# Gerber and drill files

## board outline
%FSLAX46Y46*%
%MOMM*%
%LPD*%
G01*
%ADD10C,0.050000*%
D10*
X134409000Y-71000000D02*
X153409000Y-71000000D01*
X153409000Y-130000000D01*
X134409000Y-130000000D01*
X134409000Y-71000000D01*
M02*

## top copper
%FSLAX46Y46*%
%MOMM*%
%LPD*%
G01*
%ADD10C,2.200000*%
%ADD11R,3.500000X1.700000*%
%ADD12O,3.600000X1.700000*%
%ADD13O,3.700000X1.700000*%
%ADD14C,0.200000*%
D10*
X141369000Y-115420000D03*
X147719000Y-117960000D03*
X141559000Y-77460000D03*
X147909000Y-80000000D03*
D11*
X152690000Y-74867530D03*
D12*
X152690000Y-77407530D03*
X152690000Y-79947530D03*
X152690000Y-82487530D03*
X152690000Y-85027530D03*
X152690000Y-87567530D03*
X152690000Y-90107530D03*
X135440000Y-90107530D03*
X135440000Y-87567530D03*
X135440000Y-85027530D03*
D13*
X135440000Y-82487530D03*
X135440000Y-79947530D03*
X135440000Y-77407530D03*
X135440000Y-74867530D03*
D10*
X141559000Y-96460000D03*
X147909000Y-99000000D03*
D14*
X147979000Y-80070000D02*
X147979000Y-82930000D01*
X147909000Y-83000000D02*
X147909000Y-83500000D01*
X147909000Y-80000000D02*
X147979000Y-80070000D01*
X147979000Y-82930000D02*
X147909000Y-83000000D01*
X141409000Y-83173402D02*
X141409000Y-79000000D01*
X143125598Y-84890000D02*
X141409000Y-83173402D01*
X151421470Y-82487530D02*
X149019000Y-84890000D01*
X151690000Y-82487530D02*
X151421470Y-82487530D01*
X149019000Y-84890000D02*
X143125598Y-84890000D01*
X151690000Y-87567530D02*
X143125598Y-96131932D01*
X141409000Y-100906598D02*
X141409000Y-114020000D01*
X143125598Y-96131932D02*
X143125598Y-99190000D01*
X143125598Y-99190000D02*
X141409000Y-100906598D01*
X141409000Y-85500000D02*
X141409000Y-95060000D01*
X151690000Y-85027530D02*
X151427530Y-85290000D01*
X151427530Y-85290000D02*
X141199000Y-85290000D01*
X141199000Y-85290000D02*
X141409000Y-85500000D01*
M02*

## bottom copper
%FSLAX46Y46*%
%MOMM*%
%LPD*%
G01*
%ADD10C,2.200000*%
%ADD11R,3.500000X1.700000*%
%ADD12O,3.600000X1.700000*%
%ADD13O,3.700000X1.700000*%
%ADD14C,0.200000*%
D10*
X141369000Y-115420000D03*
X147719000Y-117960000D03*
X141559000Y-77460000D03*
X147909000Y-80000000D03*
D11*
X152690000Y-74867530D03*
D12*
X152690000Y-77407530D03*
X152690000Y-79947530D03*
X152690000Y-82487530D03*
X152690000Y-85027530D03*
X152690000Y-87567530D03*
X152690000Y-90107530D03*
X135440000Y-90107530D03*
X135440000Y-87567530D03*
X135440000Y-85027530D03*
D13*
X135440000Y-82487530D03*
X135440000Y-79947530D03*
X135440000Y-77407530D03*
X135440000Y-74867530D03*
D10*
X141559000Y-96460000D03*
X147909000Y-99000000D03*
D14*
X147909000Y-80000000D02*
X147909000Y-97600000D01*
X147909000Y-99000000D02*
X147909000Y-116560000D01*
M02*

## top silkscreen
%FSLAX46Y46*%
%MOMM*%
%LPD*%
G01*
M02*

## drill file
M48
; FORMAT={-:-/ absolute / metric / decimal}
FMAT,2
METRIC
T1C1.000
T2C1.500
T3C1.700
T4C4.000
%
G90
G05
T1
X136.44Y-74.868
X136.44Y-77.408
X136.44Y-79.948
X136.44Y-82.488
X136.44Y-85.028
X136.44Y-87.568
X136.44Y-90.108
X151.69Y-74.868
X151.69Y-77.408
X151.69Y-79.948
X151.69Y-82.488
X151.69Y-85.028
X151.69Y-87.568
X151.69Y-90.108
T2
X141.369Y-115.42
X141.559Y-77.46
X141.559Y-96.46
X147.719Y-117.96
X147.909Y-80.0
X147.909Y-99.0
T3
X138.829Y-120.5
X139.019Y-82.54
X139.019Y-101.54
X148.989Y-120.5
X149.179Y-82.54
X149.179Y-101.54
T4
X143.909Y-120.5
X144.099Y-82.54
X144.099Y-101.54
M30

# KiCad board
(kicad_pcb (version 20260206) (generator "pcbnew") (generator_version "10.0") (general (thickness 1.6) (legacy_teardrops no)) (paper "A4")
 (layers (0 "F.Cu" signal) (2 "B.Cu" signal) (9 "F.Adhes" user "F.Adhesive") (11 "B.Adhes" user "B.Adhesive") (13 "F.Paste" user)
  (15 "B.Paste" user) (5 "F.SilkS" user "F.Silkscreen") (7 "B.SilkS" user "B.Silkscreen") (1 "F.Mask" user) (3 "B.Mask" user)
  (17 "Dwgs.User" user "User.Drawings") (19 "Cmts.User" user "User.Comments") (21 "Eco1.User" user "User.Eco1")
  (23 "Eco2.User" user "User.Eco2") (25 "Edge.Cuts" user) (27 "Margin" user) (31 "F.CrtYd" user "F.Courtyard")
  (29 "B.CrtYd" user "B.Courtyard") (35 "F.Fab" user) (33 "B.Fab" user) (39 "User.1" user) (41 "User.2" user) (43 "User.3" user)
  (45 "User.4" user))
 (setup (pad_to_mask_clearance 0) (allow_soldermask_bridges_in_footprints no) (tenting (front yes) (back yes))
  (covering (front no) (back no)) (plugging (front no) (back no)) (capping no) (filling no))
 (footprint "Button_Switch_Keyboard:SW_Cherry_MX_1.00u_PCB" (layer "B.Cu") (at 141.369 115.42 180)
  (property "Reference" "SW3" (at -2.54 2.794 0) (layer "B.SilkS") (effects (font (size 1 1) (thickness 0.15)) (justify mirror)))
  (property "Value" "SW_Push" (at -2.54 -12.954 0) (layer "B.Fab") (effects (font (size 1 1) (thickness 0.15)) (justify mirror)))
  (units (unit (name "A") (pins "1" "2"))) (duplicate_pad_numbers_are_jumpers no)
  (pad "" np_thru_hole circle (at -7.62 -5.08 180) (size 1.7 1.7) (drill 1.7) (layers "*.Cu" "*.Mask"))
  (pad "" np_thru_hole circle (at -2.54 -5.08 180) (size 4 4) (drill 4) (layers "*.Cu" "*.Mask"))
  (pad "" np_thru_hole circle (at 2.54 -5.08 180) (size 1.7 1.7) (drill 1.7) (layers "*.Cu" "*.Mask"))
  (pad "1" thru_hole circle (at 0 0 180) (size 2.2 2.2) (drill 1.5) (layers "*.Cu" "*.Mask") (remove_unused_layers no)
   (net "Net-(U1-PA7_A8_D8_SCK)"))
  (pad "2" thru_hole circle (at -6.35 -2.54 180) (size 2.2 2.2) (drill 1.5) (layers "*.Cu" "*.Mask") (remove_unused_layers no)
   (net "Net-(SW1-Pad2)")))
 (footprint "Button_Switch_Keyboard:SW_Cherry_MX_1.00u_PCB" (layer "B.Cu") (at 141.559 77.46 180)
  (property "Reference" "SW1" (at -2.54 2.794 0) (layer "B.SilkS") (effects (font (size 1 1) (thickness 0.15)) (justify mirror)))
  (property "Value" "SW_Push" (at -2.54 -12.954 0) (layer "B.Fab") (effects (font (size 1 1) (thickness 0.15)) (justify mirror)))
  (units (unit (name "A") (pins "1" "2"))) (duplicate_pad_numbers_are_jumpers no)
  (pad "" np_thru_hole circle (at -7.62 -5.08 180) (size 1.7 1.7) (drill 1.7) (layers "*.Cu" "*.Mask"))
  (pad "" np_thru_hole circle (at -2.54 -5.08 180) (size 4 4) (drill 4) (layers "*.Cu" "*.Mask"))
  (pad "" np_thru_hole circle (at 2.54 -5.08 180) (size 1.7 1.7) (drill 1.7) (layers "*.Cu" "*.Mask"))
  (pad "1" thru_hole circle (at 0 0 180) (size 2.2 2.2) (drill 1.5) (layers "*.Cu" "*.Mask") (remove_unused_layers no)
   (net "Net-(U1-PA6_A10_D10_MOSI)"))
  (pad "2" thru_hole circle (at -6.35 -2.54 180) (size 2.2 2.2) (drill 1.5) (layers "*.Cu" "*.Mask") (remove_unused_layers no)
   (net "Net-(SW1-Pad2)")))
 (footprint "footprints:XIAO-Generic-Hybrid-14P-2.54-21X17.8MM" (layer "B.Cu") (at 144.065 82.48753 180)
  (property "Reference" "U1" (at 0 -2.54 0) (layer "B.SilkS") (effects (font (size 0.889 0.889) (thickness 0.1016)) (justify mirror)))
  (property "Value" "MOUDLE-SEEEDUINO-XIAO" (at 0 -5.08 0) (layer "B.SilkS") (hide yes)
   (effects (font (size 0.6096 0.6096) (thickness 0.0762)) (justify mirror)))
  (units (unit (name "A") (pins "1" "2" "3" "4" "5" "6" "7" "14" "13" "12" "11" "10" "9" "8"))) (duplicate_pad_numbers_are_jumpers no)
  (pad "1" thru_hole rect (at -7.625 7.62 180) (size 3.5 1.7) (drill 1 (offset -1 0)) (layers "*.Cu" "*.Mask") (remove_unused_layers no)
   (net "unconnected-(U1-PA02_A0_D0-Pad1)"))
  (pad "2" thru_hole oval (at -7.625 5.08 180) (size 3.6 1.7) (drill 1 (offset -1 0)) (layers "*.Cu" "*.Mask") (remove_unused_layers no)
   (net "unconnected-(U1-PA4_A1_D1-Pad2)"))
  (pad "3" thru_hole oval (at -7.625 2.54 180) (size 3.6 1.7) (drill 1 (offset -1 0)) (layers "*.Cu" "*.Mask") (remove_unused_layers no)
   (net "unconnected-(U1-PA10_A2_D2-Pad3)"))
  (pad "4" thru_hole oval (at -7.625 0 180) (size 3.6 1.7) (drill 1 (offset -1 0)) (layers "*.Cu" "*.Mask") (remove_unused_layers no)
   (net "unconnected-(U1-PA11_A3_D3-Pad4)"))
  (pad "5" thru_hole oval (at -7.625 -2.54 180) (size 3.6 1.7) (drill 1 (offset -1 0)) (layers "*.Cu" "*.Mask") (remove_unused_layers no)
   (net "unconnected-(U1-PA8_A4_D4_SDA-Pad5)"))
  (pad "6" thru_hole oval (at -7.625 -5.08) (size 3.6 1.7) (drill 1 (offset 1 0)) (layers "*.Cu" "*.Mask") (remove_unused_layers no)
   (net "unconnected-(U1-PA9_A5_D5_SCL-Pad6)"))
  (pad "7" thru_hole oval (at -7.625 -7.62 180) (size 3.6 1.7) (drill 1 (offset -1 0)) (layers "*.Cu" "*.Mask") (remove_unused_layers no)
   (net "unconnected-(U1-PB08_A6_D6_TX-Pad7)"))
  (pad "8" thru_hole oval (at 7.625 -7.62 180) (size 3.6 1.7) (drill 1 (offset 1 0)) (layers "*.Cu" "*.Mask") (remove_unused_layers no)
   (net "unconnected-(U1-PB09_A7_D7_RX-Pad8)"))
  (pad "9" thru_hole oval (at 7.625 -5.08 180) (size 3.6 1.7) (drill 1 (offset 1 0)) (layers "*.Cu" "*.Mask") (remove_unused_layers no)
   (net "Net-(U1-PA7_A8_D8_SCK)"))
  (pad "10" thru_hole oval (at 7.625 -2.54 180) (size 3.6 1.7) (drill 1 (offset 1 0)) (layers "*.Cu" "*.Mask") (remove_unused_layers no)
   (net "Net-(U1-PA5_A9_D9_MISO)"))
  (pad "11" thru_hole oval (at 7.625 0 180) (size 3.7 1.7) (drill 1 (offset 1 0)) (layers "*.Cu" "*.Mask") (remove_unused_layers no)
   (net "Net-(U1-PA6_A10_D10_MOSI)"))
  (pad "12" thru_hole oval (at 7.625 2.54 180) (size 3.7 1.7) (drill 1 (offset 1 0)) (layers "*.Cu" "*.Mask") (remove_unused_layers no)
   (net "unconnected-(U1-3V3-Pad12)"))
  (pad "13" thru_hole oval (at 7.625 5.08 180) (size 3.7 1.7) (drill 1 (offset 1 0)) (layers "*.Cu" "*.Mask") (remove_unused_layers no)
   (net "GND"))
  (pad "14" thru_hole oval (at 7.625 7.62 180) (size 3.7 1.7) (drill 1 (offset 1 0)) (layers "*.Cu" "*.Mask") (remove_unused_layers no)
   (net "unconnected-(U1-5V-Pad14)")))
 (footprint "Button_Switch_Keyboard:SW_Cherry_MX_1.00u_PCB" (layer "B.Cu") (at 141.559 96.46 180)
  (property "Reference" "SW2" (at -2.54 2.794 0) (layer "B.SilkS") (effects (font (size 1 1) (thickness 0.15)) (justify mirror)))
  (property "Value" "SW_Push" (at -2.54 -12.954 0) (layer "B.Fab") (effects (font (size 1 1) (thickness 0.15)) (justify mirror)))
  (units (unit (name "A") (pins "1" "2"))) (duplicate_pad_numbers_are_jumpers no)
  (pad "" np_thru_hole circle (at -7.62 -5.08 180) (size 1.7 1.7) (drill 1.7) (layers "*.Cu" "*.Mask"))
  (pad "" np_thru_hole circle (at -2.54 -5.08 180) (size 4 4) (drill 4) (layers "*.Cu" "*.Mask"))
  (pad "" np_thru_hole circle (at 2.54 -5.08 180) (size 1.7 1.7) (drill 1.7) (layers "*.Cu" "*.Mask"))
  (pad "1" thru_hole circle (at 0 0 180) (size 2.2 2.2) (drill 1.5) (layers "*.Cu" "*.Mask") (remove_unused_layers no)
   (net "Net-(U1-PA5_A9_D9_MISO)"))
  (pad "2" thru_hole circle (at -6.35 -2.54 180) (size 2.2 2.2) (drill 1.5) (layers "*.Cu" "*.Mask") (remove_unused_layers no) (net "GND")))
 (gr_rect (start 134.409 71) (end 153.409 130) (stroke (width 0.05) (type default)) (fill no) (layer "Edge.Cuts"))
 (segment (start 147.979 80.07) (end 147.979 82.93) (width 0.2) (layer "F.Cu") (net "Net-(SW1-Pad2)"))
 (segment (start 147.909 83) (end 147.909 83.5) (width 0.2) (layer "F.Cu") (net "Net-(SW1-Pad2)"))
 (segment (start 147.909 80) (end 147.979 80.07) (width 0.2) (layer "F.Cu") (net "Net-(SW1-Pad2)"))
 (segment (start 147.979 82.93) (end 147.909 83) (width 0.2) (layer "F.Cu") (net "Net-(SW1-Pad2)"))
 (segment (start 147.909 80) (end 147.909 97.6) (width 0.2) (layer "B.Cu") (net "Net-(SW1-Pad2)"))
 (segment (start 147.909 99) (end 147.909 116.56) (width 0.2) (layer "B.Cu") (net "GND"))
 (segment (start 141.409 83.173402) (end 141.409 79) (width 0.2) (layer "F.Cu") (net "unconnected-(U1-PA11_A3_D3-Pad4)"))
 (segment (start 143.125598 84.89) (end 141.409 83.173402) (width 0.2) (layer "F.Cu") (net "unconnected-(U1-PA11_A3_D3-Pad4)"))
 (segment (start 151.42147 82.48753) (end 149.019 84.89) (width 0.2) (layer "F.Cu") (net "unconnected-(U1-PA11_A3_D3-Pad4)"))
 (segment (start 151.69 82.48753) (end 151.42147 82.48753) (width 0.2) (layer "F.Cu") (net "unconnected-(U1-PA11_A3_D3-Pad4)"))
 (segment (start 149.019 84.89) (end 143.125598 84.89) (width 0.2) (layer "F.Cu") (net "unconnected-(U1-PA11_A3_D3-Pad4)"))
 (segment (start 151.69 87.56753) (end 143.125598 96.131932) (width 0.2) (layer "F.Cu") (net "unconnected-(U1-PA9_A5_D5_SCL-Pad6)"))
 (segment (start 141.409 100.906598) (end 141.409 114.02) (width 0.2) (layer "F.Cu") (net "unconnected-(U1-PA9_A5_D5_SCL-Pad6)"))
 (segment (start 143.125598 96.131932) (end 143.125598 99.19) (width 0.2) (layer "F.Cu") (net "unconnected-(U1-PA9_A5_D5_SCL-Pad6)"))
 (segment (start 143.125598 99.19) (end 141.409 100.906598) (width 0.2) (layer "F.Cu") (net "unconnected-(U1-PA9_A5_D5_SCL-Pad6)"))
 (segment (start 141.409 85.5) (end 141.409 95.06) (width 0.2) (layer "F.Cu") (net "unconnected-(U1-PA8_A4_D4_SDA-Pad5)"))
 (segment (start 151.69 85.02753) (end 151.42753 85.29) (width 0.2) (layer "F.Cu") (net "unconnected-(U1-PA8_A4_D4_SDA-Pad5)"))
 (segment (start 151.42753 85.29) (end 141.199 85.29) (width 0.2) (layer "F.Cu") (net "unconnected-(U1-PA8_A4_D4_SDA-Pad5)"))
 (segment (start 141.199 85.29) (end 141.409 85.5) (width 0.2) (layer "F.Cu") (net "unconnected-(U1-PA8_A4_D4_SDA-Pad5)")))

